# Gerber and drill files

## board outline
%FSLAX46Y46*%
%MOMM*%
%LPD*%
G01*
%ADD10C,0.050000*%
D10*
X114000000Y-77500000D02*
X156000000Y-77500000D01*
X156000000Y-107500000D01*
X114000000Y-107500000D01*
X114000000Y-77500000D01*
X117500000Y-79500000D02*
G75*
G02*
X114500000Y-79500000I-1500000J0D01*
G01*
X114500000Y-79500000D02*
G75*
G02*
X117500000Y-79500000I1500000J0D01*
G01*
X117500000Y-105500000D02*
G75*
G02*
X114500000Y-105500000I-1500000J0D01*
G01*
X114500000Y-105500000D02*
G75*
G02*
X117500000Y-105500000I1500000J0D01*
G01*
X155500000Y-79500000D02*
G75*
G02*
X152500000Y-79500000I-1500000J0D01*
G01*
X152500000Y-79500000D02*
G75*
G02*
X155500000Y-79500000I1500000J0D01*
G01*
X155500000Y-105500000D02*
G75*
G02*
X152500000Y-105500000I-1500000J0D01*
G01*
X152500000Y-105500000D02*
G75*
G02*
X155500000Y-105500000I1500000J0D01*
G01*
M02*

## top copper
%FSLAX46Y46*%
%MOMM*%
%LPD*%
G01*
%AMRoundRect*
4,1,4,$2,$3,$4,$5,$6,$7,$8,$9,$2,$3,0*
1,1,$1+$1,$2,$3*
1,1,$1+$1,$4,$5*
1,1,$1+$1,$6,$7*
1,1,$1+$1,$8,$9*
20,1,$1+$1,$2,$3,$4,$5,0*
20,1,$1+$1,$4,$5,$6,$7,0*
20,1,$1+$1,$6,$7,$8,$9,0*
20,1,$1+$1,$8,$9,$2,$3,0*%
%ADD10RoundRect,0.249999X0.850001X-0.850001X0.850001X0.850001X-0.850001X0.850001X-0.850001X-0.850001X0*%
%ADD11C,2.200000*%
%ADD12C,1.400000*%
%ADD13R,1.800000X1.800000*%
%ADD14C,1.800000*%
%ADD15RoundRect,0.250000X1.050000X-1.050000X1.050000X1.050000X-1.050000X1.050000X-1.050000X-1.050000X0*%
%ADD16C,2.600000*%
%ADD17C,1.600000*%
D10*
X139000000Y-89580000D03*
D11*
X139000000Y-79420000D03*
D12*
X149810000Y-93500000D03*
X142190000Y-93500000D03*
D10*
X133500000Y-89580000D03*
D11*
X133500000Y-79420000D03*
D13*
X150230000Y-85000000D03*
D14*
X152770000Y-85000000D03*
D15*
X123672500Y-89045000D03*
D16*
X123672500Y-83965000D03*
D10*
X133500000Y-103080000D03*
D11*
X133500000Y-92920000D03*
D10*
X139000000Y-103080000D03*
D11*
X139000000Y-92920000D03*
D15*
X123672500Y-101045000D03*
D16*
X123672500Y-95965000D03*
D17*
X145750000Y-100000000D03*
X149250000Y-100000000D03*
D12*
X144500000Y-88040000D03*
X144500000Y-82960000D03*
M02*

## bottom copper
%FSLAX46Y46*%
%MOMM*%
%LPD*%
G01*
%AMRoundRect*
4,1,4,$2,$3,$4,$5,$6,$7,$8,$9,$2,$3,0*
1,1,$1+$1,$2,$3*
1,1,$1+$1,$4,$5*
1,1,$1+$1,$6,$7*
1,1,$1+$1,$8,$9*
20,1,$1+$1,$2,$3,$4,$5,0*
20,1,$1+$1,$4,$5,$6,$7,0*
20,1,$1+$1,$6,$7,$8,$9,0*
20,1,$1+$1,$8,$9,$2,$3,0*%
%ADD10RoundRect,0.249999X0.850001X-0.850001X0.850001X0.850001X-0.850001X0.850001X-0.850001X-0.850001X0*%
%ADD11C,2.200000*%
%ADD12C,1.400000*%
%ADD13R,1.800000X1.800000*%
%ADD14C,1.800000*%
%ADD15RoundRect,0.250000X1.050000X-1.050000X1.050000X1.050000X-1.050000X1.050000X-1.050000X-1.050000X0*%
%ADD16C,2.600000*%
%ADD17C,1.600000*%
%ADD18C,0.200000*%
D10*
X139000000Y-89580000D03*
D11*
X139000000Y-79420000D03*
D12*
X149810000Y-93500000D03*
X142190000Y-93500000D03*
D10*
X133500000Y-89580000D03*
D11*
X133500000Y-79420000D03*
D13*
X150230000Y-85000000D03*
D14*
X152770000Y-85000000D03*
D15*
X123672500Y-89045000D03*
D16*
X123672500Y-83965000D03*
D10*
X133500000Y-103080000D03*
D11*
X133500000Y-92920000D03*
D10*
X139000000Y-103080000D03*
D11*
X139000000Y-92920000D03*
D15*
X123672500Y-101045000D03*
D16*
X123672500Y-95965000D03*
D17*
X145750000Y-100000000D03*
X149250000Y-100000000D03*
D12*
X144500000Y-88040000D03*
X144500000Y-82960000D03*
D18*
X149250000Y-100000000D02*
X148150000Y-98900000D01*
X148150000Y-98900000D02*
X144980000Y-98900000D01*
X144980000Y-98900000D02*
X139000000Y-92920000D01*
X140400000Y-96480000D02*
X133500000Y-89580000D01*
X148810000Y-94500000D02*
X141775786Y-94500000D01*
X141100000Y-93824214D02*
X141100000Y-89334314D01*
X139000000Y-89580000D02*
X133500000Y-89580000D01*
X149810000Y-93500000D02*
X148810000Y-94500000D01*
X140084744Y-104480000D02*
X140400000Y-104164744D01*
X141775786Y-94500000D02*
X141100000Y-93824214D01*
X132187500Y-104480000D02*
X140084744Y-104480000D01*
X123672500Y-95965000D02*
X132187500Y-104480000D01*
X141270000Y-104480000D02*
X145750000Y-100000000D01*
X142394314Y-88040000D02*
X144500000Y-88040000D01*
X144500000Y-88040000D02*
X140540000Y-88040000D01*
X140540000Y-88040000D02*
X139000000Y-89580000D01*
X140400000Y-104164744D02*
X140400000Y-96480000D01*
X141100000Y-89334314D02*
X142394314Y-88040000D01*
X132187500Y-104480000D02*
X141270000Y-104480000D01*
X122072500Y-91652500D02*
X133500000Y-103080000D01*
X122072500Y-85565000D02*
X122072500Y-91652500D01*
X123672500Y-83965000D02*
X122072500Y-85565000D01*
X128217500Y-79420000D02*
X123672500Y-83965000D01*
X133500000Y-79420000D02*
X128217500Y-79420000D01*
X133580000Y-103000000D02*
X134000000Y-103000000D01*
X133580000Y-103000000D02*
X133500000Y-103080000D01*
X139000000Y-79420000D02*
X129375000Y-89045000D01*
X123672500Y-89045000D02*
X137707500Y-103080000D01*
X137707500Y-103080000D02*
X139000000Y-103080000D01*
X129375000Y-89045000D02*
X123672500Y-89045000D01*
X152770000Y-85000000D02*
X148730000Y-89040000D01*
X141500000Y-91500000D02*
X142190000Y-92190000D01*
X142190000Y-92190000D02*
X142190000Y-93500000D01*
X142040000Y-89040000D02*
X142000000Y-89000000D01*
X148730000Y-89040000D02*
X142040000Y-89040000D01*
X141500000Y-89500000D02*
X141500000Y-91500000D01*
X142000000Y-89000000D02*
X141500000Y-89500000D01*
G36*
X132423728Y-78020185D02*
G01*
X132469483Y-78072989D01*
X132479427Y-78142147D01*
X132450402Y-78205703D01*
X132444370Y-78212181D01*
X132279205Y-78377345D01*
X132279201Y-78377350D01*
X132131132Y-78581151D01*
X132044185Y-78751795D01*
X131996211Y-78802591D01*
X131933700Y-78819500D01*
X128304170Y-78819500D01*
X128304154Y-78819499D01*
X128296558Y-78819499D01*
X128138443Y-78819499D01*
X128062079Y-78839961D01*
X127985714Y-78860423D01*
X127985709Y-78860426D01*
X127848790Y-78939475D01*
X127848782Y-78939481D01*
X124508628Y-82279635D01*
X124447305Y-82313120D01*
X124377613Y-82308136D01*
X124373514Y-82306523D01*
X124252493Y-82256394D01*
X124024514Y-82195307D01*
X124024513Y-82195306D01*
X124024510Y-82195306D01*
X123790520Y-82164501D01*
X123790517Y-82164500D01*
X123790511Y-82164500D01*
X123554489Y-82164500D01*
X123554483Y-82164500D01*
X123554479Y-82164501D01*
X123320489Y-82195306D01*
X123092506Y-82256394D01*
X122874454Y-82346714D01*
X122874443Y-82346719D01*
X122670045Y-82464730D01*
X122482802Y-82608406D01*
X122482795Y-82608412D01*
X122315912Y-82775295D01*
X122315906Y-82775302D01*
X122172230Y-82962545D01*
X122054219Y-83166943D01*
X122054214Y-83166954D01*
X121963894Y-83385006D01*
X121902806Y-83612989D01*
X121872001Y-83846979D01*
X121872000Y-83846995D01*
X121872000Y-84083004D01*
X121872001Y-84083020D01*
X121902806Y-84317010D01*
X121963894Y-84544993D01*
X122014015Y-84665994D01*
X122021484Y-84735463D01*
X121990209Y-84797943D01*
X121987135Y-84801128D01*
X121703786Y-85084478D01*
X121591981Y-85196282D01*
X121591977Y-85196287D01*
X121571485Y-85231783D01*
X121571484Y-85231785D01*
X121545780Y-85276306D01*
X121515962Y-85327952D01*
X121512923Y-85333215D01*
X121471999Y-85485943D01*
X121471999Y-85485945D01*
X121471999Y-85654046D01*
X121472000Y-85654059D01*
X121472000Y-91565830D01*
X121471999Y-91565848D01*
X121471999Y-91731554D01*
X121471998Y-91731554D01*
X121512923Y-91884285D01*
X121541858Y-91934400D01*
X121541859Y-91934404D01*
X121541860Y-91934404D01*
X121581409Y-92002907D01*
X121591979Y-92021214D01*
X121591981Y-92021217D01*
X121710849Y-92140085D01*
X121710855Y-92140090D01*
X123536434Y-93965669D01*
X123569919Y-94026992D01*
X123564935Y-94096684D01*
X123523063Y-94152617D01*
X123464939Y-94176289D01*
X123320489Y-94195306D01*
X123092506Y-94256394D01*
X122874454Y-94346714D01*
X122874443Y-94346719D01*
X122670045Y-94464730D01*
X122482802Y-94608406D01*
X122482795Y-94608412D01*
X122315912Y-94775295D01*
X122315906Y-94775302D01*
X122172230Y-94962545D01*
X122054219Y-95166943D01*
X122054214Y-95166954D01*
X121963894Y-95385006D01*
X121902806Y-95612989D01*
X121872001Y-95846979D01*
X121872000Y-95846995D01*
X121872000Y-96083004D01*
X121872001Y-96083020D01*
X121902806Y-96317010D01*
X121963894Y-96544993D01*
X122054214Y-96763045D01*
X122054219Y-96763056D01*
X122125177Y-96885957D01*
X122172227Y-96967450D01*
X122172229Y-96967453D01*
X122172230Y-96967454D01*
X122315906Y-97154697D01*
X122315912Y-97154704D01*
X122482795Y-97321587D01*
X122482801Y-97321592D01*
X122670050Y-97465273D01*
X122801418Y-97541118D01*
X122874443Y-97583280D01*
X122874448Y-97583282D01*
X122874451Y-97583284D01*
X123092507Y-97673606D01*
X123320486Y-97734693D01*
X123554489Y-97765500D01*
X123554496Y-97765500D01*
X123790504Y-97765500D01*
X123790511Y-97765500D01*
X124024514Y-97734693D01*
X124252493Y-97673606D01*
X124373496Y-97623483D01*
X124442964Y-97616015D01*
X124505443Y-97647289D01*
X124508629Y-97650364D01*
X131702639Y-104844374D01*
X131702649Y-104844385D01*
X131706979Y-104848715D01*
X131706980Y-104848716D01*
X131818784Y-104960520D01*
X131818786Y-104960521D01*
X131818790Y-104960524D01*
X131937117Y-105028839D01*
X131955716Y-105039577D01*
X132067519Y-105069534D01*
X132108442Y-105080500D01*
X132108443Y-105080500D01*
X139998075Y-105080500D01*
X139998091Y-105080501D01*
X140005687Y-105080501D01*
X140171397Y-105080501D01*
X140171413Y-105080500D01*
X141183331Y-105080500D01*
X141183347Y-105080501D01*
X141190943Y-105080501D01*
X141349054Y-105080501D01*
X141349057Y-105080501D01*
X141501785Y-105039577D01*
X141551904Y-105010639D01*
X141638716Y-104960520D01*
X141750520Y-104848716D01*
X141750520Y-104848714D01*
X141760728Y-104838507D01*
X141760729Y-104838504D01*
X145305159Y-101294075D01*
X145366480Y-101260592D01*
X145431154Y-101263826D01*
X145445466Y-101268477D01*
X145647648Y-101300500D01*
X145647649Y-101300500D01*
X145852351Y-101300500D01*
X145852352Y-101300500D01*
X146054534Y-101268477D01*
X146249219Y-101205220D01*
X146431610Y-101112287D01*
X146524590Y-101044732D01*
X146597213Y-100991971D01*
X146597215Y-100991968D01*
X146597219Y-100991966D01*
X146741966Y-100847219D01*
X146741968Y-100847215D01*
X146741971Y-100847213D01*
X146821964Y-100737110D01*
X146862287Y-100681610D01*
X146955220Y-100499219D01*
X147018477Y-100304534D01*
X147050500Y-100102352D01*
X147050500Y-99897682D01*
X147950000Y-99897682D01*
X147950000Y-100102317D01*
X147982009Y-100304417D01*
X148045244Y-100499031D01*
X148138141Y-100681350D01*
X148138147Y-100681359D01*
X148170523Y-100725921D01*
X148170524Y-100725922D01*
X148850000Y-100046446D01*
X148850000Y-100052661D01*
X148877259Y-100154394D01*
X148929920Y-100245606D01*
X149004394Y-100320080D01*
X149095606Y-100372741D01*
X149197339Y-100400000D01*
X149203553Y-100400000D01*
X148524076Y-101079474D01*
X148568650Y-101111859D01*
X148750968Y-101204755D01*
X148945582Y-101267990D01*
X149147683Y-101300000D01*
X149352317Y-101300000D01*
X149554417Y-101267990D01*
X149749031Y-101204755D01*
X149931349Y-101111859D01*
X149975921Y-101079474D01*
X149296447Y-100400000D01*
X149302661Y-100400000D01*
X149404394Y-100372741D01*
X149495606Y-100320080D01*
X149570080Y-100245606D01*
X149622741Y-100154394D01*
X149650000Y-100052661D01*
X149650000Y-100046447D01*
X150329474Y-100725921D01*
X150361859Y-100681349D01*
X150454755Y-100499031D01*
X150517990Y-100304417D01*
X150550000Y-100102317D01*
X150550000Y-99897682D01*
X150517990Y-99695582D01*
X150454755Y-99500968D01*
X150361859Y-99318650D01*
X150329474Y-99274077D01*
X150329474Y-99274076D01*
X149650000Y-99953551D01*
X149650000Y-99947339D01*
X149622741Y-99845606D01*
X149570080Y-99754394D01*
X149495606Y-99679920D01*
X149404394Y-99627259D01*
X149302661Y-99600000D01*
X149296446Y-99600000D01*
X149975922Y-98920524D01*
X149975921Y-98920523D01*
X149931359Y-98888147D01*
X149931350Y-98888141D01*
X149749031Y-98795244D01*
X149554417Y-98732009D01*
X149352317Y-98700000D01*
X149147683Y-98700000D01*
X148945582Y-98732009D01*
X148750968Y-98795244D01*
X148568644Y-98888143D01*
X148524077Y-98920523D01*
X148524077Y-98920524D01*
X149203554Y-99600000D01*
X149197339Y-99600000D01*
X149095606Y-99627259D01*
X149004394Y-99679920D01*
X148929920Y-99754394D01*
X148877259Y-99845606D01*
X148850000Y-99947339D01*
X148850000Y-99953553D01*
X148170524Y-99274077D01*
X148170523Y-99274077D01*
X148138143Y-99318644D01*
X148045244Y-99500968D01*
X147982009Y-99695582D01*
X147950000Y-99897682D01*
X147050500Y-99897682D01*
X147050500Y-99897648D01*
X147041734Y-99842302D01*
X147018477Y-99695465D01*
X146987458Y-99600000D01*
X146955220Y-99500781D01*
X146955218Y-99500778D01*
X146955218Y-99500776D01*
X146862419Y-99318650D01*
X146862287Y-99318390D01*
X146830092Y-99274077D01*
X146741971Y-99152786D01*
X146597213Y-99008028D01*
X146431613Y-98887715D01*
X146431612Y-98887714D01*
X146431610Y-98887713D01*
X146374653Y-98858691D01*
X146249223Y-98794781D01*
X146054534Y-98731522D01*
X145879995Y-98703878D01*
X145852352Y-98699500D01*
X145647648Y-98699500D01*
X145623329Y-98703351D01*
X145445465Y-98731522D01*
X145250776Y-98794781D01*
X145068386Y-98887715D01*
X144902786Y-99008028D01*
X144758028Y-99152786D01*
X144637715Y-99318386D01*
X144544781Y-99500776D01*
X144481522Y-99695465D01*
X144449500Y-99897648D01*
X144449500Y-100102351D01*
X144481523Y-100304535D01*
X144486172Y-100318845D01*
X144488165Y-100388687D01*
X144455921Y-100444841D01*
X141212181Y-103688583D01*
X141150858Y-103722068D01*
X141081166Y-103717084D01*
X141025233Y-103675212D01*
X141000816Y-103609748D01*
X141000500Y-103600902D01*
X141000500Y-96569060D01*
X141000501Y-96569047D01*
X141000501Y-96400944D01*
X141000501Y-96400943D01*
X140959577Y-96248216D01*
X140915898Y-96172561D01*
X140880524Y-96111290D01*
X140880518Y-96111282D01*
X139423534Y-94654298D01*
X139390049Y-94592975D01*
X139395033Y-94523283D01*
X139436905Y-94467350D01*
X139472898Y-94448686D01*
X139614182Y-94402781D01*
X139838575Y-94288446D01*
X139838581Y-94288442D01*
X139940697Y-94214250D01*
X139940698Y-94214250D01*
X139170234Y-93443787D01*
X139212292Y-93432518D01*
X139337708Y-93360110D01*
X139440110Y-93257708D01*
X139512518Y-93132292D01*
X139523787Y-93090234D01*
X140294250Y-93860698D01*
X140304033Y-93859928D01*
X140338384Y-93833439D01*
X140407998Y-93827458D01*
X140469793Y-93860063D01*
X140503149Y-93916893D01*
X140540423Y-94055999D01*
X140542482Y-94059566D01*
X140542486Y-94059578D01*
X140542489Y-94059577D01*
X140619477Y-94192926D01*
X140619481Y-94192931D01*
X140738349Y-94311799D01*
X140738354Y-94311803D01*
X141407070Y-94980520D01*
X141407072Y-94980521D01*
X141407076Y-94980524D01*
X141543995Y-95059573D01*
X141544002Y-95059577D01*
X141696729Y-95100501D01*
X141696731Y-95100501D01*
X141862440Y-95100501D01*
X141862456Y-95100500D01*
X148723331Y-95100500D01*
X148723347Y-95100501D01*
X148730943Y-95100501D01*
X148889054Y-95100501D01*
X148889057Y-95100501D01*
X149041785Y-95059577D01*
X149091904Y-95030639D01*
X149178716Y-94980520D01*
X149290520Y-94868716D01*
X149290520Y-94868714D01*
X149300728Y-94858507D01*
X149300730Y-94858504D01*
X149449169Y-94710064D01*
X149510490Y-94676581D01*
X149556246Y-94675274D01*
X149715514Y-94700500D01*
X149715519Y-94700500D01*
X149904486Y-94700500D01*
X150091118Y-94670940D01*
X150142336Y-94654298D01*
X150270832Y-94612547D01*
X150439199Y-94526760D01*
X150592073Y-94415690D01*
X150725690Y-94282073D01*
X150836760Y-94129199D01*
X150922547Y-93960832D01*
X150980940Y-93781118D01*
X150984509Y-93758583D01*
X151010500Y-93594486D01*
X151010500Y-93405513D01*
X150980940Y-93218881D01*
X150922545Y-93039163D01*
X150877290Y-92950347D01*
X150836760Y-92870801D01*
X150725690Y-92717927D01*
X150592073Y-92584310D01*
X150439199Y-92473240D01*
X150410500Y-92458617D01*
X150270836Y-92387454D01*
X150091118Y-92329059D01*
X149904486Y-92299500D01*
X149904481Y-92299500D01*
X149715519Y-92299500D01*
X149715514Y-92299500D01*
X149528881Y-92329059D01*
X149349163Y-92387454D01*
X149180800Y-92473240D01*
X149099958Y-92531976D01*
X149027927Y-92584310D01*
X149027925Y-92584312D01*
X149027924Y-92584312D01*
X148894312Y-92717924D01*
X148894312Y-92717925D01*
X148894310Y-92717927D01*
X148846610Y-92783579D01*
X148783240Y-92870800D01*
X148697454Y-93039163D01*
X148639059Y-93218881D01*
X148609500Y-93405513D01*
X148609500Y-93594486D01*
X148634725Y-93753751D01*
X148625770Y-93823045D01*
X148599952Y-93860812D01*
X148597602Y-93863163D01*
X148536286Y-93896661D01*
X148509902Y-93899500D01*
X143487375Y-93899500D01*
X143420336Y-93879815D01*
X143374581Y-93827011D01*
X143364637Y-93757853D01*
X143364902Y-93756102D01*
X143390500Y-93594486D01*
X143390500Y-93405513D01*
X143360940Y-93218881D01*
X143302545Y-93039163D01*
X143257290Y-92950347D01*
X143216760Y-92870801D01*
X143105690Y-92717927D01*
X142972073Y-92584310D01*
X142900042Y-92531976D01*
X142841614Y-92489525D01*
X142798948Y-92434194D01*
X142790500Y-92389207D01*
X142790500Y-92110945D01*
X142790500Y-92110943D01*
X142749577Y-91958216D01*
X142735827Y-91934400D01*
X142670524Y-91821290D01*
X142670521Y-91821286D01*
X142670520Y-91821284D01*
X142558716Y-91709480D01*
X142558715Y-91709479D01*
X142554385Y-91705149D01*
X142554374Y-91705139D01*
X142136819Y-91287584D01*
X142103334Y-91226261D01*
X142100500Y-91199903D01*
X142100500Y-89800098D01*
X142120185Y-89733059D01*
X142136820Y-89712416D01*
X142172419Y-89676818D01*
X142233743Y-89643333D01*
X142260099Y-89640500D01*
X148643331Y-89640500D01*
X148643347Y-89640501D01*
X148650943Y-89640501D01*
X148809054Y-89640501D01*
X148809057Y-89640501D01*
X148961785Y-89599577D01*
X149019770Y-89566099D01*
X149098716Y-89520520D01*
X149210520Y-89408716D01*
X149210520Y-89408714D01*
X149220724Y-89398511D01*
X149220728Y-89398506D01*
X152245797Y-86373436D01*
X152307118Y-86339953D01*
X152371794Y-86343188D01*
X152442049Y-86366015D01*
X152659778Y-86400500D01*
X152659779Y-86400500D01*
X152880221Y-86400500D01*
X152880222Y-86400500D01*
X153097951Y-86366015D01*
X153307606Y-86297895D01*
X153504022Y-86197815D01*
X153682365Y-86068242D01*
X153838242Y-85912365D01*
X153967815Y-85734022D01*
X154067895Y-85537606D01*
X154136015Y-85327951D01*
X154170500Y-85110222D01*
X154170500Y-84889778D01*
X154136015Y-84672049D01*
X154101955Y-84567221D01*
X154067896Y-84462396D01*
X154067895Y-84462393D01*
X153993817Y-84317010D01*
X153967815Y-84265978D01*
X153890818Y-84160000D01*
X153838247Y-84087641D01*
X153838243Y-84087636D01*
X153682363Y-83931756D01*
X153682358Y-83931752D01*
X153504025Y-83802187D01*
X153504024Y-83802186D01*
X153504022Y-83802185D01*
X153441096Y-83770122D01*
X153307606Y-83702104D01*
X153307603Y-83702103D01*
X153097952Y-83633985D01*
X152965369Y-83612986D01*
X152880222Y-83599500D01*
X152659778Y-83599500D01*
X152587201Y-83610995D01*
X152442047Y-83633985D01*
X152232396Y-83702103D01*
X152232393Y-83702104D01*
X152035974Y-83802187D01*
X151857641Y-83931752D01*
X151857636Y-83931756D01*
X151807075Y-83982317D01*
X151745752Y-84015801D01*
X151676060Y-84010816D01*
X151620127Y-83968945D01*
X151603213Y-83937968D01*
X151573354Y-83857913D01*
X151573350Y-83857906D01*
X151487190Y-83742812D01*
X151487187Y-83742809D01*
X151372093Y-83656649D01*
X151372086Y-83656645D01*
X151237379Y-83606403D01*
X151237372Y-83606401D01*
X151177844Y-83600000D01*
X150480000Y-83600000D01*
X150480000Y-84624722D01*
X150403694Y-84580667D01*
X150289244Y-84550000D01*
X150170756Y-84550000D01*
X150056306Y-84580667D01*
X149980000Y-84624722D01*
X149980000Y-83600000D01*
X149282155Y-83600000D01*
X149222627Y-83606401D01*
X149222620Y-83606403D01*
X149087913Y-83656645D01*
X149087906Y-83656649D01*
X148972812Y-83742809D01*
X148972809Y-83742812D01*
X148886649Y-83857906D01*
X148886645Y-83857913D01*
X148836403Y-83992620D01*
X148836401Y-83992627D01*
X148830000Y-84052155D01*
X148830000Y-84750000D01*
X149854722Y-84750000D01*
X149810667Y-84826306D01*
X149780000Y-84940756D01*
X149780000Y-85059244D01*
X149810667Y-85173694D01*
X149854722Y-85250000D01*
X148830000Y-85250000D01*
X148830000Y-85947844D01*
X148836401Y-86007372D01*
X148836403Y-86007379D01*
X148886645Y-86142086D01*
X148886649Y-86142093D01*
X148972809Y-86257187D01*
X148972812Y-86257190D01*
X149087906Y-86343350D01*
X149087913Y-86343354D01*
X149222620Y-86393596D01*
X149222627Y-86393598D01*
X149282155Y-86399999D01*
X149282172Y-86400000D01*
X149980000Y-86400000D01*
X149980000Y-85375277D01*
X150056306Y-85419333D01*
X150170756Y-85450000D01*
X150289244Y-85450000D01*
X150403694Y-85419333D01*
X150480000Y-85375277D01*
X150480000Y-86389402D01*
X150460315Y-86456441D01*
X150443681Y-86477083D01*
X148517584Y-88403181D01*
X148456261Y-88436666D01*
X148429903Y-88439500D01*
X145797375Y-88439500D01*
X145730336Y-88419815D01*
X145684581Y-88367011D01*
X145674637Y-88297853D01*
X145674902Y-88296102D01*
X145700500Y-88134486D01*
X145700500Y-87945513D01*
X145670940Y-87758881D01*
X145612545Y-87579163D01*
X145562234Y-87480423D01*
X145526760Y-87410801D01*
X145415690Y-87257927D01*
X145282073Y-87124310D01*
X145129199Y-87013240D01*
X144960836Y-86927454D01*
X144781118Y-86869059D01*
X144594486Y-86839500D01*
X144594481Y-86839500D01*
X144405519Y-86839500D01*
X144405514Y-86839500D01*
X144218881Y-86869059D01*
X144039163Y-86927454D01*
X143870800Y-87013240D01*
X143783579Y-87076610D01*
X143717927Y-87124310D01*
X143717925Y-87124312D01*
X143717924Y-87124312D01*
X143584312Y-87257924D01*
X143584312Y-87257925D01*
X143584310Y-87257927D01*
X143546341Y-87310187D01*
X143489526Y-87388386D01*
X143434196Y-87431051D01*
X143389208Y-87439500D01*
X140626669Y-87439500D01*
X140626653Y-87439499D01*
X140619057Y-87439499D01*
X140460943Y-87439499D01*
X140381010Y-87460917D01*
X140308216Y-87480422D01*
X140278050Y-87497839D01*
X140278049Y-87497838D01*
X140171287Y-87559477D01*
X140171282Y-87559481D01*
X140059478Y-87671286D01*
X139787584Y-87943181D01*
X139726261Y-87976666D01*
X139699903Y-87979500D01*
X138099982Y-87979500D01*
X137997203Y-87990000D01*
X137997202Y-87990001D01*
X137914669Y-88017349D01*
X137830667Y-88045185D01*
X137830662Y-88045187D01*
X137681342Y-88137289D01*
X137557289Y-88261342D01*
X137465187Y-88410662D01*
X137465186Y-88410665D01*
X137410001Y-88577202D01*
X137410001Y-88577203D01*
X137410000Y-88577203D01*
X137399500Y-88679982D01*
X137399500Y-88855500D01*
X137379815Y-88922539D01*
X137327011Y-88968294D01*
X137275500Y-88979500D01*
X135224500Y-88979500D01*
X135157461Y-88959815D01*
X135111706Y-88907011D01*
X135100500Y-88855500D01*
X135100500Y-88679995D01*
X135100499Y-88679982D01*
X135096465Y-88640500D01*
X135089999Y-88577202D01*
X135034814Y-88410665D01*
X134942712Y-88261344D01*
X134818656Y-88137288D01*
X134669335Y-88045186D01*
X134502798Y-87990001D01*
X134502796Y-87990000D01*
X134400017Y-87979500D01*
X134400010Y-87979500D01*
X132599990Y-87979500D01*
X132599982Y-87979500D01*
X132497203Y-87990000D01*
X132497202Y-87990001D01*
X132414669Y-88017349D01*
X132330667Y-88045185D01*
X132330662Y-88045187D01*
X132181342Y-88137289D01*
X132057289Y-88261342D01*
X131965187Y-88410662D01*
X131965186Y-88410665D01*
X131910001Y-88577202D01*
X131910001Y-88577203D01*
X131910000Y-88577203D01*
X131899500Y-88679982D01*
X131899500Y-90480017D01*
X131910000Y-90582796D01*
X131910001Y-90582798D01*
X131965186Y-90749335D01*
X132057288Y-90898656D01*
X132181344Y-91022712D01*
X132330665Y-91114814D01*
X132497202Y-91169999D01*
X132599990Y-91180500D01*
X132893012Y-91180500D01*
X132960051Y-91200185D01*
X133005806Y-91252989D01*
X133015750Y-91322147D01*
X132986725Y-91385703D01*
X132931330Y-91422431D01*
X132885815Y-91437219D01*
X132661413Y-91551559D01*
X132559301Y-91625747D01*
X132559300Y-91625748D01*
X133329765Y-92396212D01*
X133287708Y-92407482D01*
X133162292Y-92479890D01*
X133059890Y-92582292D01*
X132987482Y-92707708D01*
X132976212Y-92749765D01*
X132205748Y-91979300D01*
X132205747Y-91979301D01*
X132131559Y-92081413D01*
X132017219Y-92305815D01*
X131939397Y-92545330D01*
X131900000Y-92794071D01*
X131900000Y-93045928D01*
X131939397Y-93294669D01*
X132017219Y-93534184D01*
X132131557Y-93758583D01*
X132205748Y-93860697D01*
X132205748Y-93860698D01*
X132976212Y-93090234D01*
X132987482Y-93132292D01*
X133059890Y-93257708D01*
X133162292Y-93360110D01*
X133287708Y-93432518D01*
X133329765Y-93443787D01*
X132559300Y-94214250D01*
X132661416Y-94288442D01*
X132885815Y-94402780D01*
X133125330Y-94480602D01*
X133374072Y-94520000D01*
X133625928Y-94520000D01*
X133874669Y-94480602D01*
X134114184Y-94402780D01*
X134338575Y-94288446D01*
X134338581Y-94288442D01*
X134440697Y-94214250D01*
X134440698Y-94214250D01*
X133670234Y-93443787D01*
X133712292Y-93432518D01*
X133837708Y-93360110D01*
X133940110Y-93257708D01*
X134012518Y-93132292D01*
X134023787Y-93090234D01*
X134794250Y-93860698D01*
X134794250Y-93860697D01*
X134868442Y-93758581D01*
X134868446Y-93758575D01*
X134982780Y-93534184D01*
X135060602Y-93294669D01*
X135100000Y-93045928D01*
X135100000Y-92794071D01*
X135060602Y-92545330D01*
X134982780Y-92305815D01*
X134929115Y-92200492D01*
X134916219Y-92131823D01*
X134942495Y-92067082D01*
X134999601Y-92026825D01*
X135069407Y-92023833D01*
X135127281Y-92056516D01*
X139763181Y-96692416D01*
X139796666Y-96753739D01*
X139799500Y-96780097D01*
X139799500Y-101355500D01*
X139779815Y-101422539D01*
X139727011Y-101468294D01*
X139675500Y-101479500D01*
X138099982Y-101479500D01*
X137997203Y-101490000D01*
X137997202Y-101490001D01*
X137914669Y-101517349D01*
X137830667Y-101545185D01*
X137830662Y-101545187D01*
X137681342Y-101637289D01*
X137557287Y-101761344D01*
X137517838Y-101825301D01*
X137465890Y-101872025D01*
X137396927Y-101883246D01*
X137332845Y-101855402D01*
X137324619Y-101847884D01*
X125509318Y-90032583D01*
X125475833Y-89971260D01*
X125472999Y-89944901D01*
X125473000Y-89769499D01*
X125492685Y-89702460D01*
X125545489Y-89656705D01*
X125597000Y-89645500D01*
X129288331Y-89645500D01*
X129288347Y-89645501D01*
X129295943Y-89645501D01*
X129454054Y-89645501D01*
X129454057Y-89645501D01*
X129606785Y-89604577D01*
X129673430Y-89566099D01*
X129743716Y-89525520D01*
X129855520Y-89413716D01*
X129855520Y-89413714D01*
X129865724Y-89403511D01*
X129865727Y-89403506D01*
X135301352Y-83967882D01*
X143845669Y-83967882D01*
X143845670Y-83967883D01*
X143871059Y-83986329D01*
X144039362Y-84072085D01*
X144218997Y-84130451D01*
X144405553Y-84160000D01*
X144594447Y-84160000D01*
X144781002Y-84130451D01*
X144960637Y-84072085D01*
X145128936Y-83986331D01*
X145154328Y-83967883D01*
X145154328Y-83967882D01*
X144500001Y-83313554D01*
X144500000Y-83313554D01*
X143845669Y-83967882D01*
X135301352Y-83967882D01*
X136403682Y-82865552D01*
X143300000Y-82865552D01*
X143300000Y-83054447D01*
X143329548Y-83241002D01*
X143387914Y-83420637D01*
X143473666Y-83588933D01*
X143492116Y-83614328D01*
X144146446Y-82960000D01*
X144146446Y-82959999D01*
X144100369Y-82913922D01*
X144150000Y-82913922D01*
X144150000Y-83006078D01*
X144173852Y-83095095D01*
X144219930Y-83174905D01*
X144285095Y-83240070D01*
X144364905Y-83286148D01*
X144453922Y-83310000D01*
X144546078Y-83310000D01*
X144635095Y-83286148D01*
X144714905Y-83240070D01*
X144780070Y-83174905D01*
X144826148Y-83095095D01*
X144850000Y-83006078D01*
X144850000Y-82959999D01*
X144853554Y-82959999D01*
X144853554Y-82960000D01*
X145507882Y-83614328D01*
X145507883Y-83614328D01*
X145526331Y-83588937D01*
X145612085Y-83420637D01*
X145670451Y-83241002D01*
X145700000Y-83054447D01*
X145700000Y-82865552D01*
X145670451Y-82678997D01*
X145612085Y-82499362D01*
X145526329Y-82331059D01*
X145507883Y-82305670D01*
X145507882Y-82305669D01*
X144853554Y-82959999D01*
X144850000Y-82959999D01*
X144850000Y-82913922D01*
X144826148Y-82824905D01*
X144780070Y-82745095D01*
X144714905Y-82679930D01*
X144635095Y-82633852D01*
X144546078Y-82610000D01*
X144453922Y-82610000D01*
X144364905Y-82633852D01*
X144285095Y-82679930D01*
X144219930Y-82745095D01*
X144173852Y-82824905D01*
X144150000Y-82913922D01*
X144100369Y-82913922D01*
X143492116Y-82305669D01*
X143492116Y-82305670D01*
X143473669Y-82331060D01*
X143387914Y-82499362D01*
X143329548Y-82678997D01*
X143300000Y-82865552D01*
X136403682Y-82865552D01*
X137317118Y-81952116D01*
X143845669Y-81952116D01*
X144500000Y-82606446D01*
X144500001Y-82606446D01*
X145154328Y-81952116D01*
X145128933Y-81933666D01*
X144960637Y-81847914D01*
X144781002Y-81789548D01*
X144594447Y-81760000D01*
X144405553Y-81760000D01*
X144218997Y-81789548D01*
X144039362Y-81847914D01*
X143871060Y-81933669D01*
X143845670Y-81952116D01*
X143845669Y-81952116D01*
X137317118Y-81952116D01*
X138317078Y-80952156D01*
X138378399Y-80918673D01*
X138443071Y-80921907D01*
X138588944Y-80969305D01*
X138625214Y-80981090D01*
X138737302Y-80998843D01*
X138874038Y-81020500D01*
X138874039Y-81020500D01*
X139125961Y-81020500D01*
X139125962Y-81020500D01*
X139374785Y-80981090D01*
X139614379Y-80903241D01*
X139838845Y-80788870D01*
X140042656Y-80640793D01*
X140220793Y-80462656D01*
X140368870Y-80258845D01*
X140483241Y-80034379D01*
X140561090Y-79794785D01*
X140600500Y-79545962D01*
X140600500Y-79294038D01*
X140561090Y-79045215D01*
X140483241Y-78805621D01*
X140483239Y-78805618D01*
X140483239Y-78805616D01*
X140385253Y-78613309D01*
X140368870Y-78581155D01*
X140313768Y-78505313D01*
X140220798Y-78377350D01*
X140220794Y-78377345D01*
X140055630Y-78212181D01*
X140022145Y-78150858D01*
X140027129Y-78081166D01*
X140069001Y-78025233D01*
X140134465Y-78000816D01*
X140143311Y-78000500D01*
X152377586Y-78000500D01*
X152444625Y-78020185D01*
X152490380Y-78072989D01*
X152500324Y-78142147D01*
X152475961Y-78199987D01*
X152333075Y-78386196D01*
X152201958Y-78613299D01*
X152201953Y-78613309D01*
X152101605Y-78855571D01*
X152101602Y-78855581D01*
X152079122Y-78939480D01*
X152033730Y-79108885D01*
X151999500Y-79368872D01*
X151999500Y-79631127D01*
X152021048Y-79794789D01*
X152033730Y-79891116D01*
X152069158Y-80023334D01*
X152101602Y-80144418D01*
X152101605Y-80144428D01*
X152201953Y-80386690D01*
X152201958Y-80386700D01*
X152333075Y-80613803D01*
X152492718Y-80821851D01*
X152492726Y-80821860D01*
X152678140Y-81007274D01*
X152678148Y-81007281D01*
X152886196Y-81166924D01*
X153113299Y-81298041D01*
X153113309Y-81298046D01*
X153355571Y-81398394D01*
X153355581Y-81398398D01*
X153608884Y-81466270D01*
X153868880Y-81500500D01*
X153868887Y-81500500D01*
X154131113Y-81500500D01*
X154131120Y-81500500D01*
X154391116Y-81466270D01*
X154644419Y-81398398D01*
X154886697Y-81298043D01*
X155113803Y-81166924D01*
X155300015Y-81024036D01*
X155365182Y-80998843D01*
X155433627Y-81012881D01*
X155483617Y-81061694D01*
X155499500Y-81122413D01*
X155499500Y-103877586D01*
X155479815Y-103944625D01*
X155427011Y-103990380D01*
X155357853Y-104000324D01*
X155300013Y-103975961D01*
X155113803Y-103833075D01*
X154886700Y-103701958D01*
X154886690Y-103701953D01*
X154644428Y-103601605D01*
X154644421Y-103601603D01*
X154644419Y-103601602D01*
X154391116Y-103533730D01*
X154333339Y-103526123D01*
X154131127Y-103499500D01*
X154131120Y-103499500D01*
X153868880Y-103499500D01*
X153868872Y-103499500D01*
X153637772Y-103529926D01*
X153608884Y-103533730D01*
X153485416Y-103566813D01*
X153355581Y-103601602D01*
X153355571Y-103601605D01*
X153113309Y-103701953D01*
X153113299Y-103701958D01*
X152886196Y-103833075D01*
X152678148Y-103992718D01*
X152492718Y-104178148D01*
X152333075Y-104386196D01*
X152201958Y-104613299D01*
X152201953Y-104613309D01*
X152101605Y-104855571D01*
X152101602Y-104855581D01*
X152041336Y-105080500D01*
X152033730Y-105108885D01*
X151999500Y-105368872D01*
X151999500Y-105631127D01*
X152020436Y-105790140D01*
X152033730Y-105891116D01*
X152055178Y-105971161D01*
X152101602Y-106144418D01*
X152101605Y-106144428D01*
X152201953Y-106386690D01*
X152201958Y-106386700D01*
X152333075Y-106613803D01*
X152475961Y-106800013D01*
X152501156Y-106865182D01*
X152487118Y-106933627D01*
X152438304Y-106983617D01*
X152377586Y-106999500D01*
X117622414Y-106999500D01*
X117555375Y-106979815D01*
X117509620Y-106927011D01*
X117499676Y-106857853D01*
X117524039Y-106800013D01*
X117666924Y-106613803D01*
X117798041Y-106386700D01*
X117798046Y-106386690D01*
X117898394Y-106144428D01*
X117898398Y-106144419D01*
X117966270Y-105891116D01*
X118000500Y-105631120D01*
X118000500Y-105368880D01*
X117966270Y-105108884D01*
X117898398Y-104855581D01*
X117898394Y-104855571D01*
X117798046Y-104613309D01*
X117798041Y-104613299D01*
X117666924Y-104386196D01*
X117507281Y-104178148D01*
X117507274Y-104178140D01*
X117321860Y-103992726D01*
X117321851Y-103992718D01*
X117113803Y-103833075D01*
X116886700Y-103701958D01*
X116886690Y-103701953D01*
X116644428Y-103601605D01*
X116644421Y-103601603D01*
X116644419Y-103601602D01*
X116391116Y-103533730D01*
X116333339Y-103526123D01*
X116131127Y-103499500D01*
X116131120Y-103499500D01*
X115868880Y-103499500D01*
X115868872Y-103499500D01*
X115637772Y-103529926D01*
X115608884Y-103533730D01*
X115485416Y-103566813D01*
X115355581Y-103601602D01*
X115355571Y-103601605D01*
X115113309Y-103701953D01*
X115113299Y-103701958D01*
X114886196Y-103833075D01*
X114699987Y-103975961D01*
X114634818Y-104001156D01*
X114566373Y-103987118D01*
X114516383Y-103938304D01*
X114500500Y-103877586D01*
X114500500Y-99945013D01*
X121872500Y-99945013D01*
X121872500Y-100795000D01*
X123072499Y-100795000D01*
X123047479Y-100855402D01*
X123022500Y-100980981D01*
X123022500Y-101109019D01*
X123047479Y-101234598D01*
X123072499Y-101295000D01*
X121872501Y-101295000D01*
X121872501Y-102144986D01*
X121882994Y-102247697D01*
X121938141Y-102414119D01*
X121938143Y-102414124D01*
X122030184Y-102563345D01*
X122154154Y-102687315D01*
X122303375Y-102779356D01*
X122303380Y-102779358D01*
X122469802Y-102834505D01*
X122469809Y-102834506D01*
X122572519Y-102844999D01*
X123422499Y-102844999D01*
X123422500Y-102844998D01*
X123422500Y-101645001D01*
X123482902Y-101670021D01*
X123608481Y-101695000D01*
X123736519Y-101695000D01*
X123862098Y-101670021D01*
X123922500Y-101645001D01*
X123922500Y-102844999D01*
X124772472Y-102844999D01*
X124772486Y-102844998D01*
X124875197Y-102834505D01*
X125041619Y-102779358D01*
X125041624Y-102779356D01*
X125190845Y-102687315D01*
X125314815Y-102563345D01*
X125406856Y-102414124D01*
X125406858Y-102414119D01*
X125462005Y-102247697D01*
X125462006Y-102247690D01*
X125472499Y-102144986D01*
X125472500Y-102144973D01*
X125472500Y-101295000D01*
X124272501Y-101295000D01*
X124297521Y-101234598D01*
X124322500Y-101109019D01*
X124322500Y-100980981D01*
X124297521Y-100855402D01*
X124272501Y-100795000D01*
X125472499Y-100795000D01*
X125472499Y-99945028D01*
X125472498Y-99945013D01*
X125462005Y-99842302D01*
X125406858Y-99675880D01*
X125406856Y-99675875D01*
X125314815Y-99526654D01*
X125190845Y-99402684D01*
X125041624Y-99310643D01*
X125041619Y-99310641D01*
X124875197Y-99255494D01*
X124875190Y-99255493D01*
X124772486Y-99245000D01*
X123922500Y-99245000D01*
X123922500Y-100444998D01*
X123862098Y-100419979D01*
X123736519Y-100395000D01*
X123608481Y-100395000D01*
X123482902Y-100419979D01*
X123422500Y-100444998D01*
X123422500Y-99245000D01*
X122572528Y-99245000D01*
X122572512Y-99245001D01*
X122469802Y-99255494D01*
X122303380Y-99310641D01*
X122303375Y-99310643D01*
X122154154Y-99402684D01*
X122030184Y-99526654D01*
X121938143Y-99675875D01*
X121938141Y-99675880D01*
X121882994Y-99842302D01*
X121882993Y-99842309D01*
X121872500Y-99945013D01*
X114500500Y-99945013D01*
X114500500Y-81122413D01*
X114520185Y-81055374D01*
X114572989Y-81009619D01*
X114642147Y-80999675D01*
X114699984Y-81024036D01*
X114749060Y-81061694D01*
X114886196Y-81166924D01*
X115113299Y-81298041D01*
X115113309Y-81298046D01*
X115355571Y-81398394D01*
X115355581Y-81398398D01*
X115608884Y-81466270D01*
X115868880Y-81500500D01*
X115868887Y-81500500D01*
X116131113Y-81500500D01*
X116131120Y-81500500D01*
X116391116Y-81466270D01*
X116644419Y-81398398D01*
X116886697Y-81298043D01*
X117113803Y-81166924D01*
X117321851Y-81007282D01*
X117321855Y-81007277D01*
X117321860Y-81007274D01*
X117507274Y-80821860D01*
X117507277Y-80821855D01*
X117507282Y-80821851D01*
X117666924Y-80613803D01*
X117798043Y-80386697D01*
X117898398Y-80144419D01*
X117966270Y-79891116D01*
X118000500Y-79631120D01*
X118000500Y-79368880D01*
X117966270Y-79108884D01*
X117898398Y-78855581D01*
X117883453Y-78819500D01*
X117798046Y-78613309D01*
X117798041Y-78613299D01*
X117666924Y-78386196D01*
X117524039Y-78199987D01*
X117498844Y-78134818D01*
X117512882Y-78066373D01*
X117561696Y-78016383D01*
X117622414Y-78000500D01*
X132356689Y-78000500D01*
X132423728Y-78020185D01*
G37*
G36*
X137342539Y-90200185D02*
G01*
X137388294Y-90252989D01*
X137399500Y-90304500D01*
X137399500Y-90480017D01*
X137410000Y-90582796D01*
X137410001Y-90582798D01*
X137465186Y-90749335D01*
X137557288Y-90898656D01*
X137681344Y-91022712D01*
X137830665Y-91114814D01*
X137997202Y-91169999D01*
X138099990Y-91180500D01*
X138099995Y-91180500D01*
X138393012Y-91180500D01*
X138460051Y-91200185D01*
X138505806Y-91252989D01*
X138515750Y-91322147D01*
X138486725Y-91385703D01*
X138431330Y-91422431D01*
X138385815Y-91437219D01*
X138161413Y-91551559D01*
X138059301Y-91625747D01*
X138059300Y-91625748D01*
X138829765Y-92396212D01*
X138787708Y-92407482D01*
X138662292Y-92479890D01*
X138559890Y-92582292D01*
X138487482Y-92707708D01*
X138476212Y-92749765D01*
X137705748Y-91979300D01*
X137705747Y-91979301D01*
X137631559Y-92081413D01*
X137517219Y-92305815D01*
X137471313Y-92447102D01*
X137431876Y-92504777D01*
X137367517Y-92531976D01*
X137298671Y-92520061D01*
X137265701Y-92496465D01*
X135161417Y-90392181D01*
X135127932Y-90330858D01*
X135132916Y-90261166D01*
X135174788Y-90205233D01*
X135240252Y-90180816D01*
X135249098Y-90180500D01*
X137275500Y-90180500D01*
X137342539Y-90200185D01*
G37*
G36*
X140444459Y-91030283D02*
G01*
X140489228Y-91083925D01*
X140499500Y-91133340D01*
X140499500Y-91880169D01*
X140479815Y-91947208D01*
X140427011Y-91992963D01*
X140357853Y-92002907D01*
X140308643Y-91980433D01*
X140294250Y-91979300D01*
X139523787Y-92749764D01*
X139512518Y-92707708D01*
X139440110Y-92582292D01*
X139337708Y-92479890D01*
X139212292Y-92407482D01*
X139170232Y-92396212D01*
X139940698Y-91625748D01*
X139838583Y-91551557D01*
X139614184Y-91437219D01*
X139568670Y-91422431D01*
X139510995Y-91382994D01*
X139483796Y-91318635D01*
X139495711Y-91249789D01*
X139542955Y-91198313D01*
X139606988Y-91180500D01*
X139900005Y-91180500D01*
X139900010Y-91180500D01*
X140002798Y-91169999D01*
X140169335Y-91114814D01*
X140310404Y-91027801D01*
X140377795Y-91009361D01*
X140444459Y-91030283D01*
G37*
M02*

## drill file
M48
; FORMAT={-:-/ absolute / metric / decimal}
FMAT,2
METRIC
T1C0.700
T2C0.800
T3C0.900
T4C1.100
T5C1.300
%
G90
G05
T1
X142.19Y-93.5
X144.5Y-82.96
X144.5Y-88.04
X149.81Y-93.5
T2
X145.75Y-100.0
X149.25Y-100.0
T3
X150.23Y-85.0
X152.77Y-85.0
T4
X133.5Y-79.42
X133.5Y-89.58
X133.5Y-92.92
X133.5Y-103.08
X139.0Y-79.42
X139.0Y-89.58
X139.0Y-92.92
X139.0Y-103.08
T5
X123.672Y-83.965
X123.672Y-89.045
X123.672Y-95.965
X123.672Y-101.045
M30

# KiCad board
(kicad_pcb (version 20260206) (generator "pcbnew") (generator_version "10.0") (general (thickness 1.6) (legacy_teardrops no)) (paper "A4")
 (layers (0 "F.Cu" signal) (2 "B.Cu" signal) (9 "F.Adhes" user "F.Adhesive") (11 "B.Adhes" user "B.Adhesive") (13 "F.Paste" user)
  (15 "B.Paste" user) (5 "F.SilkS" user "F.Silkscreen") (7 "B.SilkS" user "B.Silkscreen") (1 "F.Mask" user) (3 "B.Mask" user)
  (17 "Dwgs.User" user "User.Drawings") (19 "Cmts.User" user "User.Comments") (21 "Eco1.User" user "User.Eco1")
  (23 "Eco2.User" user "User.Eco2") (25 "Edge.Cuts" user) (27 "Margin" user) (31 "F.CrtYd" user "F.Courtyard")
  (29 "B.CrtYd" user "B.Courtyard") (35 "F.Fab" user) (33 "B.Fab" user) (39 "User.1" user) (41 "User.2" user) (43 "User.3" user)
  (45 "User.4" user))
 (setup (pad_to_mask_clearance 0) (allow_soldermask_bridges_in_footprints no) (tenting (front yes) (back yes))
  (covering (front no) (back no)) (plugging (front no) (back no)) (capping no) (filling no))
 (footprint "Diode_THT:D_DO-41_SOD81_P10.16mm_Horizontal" (layer "F.Cu") (at 139 89.58 90)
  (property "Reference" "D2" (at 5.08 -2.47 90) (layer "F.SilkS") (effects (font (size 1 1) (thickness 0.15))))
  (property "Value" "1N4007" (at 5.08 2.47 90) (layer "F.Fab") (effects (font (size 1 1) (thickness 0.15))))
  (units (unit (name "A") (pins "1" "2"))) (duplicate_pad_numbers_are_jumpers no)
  (pad "1" thru_hole roundrect (at 0 0 90) (size 2.2 2.2) (drill 1.1) (layers "*.Cu" "*.Mask") (remove_unused_layers no)
   (roundrect_rratio 0.113636) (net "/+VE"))
  (pad "2" thru_hole circle (at 10.16 0 90) (size 2.2 2.2) (drill 1.1) (layers "*.Cu" "*.Mask") (remove_unused_layers no) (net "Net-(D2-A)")))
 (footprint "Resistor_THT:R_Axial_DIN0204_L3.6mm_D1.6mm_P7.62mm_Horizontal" (layer "F.Cu") (at 149.81 93.5 180)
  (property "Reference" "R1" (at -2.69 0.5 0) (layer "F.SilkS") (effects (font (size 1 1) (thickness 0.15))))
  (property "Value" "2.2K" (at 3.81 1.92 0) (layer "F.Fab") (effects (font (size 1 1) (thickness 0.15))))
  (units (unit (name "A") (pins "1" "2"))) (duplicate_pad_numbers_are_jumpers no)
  (pad "1" thru_hole circle (at 0 0 180) (size 1.4 1.4) (drill 0.7) (layers "*.Cu" "*.Mask") (remove_unused_layers no) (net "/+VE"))
  (pad "2" thru_hole circle (at 7.62 0 180) (size 1.4 1.4) (drill 0.7) (layers "*.Cu" "*.Mask") (remove_unused_layers no) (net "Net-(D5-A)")))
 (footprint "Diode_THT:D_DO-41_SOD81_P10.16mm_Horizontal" (layer "F.Cu") (at 133.5 89.58 90)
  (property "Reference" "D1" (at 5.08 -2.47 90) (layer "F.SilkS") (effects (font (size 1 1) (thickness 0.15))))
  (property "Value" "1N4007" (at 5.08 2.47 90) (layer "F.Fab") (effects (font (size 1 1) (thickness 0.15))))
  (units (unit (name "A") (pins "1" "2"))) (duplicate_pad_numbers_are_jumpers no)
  (pad "1" thru_hole roundrect (at 0 0 90) (size 2.2 2.2) (drill 1.1) (layers "*.Cu" "*.Mask") (remove_unused_layers no)
   (roundrect_rratio 0.113636) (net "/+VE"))
  (pad "2" thru_hole circle (at 10.16 0 90) (size 2.2 2.2) (drill 1.1) (layers "*.Cu" "*.Mask") (remove_unused_layers no) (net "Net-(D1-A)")))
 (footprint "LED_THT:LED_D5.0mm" (layer "F.Cu") (at 150.23 85)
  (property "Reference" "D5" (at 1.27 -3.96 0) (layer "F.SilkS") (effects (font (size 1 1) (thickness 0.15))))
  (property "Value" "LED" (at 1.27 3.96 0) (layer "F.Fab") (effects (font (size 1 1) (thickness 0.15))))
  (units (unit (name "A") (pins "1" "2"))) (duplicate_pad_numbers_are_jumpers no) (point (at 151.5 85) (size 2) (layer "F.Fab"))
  (pad "1" thru_hole rect (at 0 0) (size 1.8 1.8) (drill 0.9) (layers "*.Cu" "*.Mask") (remove_unused_layers no) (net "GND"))
  (pad "2" thru_hole circle (at 2.54 0) (size 1.8 1.8) (drill 0.9) (layers "*.Cu" "*.Mask") (remove_unused_layers no) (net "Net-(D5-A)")))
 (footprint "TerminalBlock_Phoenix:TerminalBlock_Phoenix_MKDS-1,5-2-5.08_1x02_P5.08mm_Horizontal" (layer "F.Cu") (at 123.6725 89.045 90)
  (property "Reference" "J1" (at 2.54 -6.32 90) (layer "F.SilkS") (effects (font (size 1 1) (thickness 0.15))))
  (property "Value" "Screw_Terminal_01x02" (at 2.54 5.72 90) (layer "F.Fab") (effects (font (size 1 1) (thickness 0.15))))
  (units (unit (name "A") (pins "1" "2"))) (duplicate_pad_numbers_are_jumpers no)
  (pad "1" thru_hole roundrect (at 0 0 90) (size 2.6 2.6) (drill 1.3) (layers "*.Cu" "*.Mask") (remove_unused_layers no)
   (roundrect_rratio 0.096154) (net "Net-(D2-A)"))
  (pad "2" thru_hole circle (at 5.08 0 90) (size 2.6 2.6) (drill 1.3) (layers "*.Cu" "*.Mask") (remove_unused_layers no) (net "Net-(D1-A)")))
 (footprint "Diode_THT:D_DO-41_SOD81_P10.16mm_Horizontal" (layer "F.Cu") (at 133.5 103.08 90)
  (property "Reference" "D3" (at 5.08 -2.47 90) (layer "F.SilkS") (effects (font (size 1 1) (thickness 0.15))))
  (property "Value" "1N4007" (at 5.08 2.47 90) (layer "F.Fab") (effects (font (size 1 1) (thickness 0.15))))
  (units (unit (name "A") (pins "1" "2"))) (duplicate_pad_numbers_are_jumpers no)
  (pad "1" thru_hole roundrect (at 0 0 90) (size 2.2 2.2) (drill 1.1) (layers "*.Cu" "*.Mask") (remove_unused_layers no)
   (roundrect_rratio 0.113636) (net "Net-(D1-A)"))
  (pad "2" thru_hole circle (at 10.16 0 90) (size 2.2 2.2) (drill 1.1) (layers "*.Cu" "*.Mask") (remove_unused_layers no) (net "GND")))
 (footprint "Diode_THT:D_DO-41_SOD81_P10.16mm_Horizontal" (layer "F.Cu") (at 139 103.08 90)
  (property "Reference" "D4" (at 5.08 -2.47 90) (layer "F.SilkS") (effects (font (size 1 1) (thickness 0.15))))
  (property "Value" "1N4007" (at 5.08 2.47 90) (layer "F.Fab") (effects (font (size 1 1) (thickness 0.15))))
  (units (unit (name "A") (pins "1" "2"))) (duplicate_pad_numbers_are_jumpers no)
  (pad "1" thru_hole roundrect (at 0 0 90) (size 2.2 2.2) (drill 1.1) (layers "*.Cu" "*.Mask") (remove_unused_layers no)
   (roundrect_rratio 0.113636) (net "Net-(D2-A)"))
  (pad "2" thru_hole circle (at 10.16 0 90) (size 2.2 2.2) (drill 1.1) (layers "*.Cu" "*.Mask") (remove_unused_layers no) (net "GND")))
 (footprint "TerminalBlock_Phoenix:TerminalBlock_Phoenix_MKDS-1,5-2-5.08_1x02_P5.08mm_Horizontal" (layer "F.Cu") (at 123.6725 101.045 90)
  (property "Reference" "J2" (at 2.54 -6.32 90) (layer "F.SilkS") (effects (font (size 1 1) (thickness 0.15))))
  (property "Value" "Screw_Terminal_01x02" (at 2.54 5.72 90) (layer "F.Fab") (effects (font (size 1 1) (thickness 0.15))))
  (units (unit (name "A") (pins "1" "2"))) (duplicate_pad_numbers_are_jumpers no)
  (pad "1" thru_hole roundrect (at 0 0 90) (size 2.6 2.6) (drill 1.3) (layers "*.Cu" "*.Mask") (remove_unused_layers no)
   (roundrect_rratio 0.096154) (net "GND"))
  (pad "2" thru_hole circle (at 5.08 0 90) (size 2.6 2.6) (drill 1.3) (layers "*.Cu" "*.Mask") (remove_unused_layers no) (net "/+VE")))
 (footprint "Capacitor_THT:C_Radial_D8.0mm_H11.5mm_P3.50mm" (layer "F.Cu") (at 145.75 100)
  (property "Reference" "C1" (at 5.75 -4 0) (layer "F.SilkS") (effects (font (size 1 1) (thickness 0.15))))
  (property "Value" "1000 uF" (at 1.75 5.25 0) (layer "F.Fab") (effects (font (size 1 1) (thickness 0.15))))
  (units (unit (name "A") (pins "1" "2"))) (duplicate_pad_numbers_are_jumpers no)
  (pad "1" thru_hole circle (at 0 0) (size 1.6 1.6) (drill 0.8) (layers "*.Cu" "*.Mask") (remove_unused_layers no) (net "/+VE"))
  (pad "2" thru_hole circle (at 3.5 0) (size 1.6 1.6) (drill 0.8) (layers "*.Cu" "*.Mask") (remove_unused_layers no) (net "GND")))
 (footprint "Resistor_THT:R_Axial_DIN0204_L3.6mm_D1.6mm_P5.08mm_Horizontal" (layer "F.Cu") (at 144.5 88.04 90)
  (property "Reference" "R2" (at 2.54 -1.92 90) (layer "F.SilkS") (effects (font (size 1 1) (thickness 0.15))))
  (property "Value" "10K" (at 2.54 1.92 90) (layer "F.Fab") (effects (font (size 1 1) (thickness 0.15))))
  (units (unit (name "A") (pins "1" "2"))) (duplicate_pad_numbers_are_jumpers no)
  (pad "1" thru_hole circle (at 0 0 90) (size 1.4 1.4) (drill 0.7) (layers "*.Cu" "*.Mask") (remove_unused_layers no) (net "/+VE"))
  (pad "2" thru_hole circle (at 5.08 0 90) (size 1.4 1.4) (drill 0.7) (layers "*.Cu" "*.Mask") (remove_unused_layers no) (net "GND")))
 (gr_rect (start 114 77.5) (end 156 107.5) (stroke (width 0.05) (type default)) (fill no) (layer "Edge.Cuts"))
 (gr_circle (center 116 79.5) (end 117.5 79.5) (stroke (width 0.05) (type default)) (fill no) (layer "Edge.Cuts"))
 (gr_circle (center 116 105.5) (end 117.5 105.5) (stroke (width 0.05) (type default)) (fill no) (layer "Edge.Cuts"))
 (gr_circle (center 154 79.5) (end 155.5 79.5) (stroke (width 0.05) (type default)) (fill no) (layer "Edge.Cuts"))
 (gr_circle (center 154 105.5) (end 155.5 105.5) (stroke (width 0.05) (type default)) (fill no) (layer "Edge.Cuts"))
 (segment (start 149.25 100) (end 148.15 98.9) (width 0.2) (layer "B.Cu") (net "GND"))
 (segment (start 148.15 98.9) (end 144.98 98.9) (width 0.2) (layer "B.Cu") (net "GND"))
 (segment (start 144.98 98.9) (end 139 92.92) (width 0.2) (layer "B.Cu") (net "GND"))
 (segment (start 140.4 96.48) (end 133.5 89.58) (width 0.2) (layer "B.Cu") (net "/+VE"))
 (segment (start 148.81 94.5) (end 141.775786 94.5) (width 0.2) (layer "B.Cu") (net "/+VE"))
 (segment (start 141.1 93.824214) (end 141.1 89.334314) (width 0.2) (layer "B.Cu") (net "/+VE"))
 (segment (start 139 89.58) (end 133.5 89.58) (width 0.2) (layer "B.Cu") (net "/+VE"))
 (segment (start 149.81 93.5) (end 148.81 94.5) (width 0.2) (layer "B.Cu") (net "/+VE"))
 (segment (start 140.084744 104.48) (end 140.4 104.164744) (width 0.2) (layer "B.Cu") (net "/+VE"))
 (segment (start 141.775786 94.5) (end 141.1 93.824214) (width 0.2) (layer "B.Cu") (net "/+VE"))
 (segment (start 132.1875 104.48) (end 140.084744 104.48) (width 0.2) (layer "B.Cu") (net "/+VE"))
 (segment (start 123.6725 95.965) (end 132.1875 104.48) (width 0.2) (layer "B.Cu") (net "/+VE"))
 (segment (start 141.27 104.48) (end 145.75 100) (width 0.2) (layer "B.Cu") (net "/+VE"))
 (segment (start 142.394314 88.04) (end 144.5 88.04) (width 0.2) (layer "B.Cu") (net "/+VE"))
 (segment (start 144.5 88.04) (end 140.54 88.04) (width 0.2) (layer "B.Cu") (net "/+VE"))
 (segment (start 140.54 88.04) (end 139 89.58) (width 0.2) (layer "B.Cu") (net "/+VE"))
 (segment (start 140.4 104.164744) (end 140.4 96.48) (width 0.2) (layer "B.Cu") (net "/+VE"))
 (segment (start 141.1 89.334314) (end 142.394314 88.04) (width 0.2) (layer "B.Cu") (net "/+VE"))
 (segment (start 132.1875 104.48) (end 141.27 104.48) (width 0.2) (layer "B.Cu") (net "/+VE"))
 (segment (start 122.0725 91.6525) (end 133.5 103.08) (width 0.2) (layer "B.Cu") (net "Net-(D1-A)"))
 (segment (start 122.0725 85.565) (end 122.0725 91.6525) (width 0.2) (layer "B.Cu") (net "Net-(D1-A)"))
 (segment (start 123.6725 83.965) (end 122.0725 85.565) (width 0.2) (layer "B.Cu") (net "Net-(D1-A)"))
 (segment (start 128.2175 79.42) (end 123.6725 83.965) (width 0.2) (layer "B.Cu") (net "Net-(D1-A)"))
 (segment (start 133.5 79.42) (end 128.2175 79.42) (width 0.2) (layer "B.Cu") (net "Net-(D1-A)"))
 (segment (start 133.58 103) (end 134 103) (width 0.2) (layer "B.Cu") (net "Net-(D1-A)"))
 (segment (start 133.58 103) (end 133.5 103.08) (width 0.2) (layer "B.Cu") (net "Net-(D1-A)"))
 (segment (start 139 79.42) (end 129.375 89.045) (width 0.2) (layer "B.Cu") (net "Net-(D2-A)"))
 (segment (start 123.6725 89.045) (end 137.7075 103.08) (width 0.2) (layer "B.Cu") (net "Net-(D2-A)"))
 (segment (start 137.7075 103.08) (end 139 103.08) (width 0.2) (layer "B.Cu") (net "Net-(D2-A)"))
 (segment (start 129.375 89.045) (end 123.6725 89.045) (width 0.2) (layer "B.Cu") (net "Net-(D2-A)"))
 (segment (start 152.77 85) (end 148.73 89.04) (width 0.2) (layer "B.Cu") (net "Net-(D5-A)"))
 (segment (start 141.5 91.5) (end 142.19 92.19) (width 0.2) (layer "B.Cu") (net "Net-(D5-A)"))
 (segment (start 142.19 92.19) (end 142.19 93.5) (width 0.2) (layer "B.Cu") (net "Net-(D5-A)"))
 (segment (start 142.04 89.04) (end 142 89) (width 0.2) (layer "B.Cu") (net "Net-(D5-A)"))
 (segment (start 148.73 89.04) (end 142.04 89.04) (width 0.2) (layer "B.Cu") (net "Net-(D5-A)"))
 (segment (start 141.5 89.5) (end 141.5 91.5) (width 0.2) (layer "B.Cu") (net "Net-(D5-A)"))
 (segment (start 142 89) (end 141.5 89.5) (width 0.2) (layer "B.Cu") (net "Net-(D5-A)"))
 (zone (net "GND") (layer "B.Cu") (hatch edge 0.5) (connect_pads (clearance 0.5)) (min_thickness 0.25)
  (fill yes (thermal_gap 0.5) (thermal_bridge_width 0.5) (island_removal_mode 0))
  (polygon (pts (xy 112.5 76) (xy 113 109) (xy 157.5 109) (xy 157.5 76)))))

